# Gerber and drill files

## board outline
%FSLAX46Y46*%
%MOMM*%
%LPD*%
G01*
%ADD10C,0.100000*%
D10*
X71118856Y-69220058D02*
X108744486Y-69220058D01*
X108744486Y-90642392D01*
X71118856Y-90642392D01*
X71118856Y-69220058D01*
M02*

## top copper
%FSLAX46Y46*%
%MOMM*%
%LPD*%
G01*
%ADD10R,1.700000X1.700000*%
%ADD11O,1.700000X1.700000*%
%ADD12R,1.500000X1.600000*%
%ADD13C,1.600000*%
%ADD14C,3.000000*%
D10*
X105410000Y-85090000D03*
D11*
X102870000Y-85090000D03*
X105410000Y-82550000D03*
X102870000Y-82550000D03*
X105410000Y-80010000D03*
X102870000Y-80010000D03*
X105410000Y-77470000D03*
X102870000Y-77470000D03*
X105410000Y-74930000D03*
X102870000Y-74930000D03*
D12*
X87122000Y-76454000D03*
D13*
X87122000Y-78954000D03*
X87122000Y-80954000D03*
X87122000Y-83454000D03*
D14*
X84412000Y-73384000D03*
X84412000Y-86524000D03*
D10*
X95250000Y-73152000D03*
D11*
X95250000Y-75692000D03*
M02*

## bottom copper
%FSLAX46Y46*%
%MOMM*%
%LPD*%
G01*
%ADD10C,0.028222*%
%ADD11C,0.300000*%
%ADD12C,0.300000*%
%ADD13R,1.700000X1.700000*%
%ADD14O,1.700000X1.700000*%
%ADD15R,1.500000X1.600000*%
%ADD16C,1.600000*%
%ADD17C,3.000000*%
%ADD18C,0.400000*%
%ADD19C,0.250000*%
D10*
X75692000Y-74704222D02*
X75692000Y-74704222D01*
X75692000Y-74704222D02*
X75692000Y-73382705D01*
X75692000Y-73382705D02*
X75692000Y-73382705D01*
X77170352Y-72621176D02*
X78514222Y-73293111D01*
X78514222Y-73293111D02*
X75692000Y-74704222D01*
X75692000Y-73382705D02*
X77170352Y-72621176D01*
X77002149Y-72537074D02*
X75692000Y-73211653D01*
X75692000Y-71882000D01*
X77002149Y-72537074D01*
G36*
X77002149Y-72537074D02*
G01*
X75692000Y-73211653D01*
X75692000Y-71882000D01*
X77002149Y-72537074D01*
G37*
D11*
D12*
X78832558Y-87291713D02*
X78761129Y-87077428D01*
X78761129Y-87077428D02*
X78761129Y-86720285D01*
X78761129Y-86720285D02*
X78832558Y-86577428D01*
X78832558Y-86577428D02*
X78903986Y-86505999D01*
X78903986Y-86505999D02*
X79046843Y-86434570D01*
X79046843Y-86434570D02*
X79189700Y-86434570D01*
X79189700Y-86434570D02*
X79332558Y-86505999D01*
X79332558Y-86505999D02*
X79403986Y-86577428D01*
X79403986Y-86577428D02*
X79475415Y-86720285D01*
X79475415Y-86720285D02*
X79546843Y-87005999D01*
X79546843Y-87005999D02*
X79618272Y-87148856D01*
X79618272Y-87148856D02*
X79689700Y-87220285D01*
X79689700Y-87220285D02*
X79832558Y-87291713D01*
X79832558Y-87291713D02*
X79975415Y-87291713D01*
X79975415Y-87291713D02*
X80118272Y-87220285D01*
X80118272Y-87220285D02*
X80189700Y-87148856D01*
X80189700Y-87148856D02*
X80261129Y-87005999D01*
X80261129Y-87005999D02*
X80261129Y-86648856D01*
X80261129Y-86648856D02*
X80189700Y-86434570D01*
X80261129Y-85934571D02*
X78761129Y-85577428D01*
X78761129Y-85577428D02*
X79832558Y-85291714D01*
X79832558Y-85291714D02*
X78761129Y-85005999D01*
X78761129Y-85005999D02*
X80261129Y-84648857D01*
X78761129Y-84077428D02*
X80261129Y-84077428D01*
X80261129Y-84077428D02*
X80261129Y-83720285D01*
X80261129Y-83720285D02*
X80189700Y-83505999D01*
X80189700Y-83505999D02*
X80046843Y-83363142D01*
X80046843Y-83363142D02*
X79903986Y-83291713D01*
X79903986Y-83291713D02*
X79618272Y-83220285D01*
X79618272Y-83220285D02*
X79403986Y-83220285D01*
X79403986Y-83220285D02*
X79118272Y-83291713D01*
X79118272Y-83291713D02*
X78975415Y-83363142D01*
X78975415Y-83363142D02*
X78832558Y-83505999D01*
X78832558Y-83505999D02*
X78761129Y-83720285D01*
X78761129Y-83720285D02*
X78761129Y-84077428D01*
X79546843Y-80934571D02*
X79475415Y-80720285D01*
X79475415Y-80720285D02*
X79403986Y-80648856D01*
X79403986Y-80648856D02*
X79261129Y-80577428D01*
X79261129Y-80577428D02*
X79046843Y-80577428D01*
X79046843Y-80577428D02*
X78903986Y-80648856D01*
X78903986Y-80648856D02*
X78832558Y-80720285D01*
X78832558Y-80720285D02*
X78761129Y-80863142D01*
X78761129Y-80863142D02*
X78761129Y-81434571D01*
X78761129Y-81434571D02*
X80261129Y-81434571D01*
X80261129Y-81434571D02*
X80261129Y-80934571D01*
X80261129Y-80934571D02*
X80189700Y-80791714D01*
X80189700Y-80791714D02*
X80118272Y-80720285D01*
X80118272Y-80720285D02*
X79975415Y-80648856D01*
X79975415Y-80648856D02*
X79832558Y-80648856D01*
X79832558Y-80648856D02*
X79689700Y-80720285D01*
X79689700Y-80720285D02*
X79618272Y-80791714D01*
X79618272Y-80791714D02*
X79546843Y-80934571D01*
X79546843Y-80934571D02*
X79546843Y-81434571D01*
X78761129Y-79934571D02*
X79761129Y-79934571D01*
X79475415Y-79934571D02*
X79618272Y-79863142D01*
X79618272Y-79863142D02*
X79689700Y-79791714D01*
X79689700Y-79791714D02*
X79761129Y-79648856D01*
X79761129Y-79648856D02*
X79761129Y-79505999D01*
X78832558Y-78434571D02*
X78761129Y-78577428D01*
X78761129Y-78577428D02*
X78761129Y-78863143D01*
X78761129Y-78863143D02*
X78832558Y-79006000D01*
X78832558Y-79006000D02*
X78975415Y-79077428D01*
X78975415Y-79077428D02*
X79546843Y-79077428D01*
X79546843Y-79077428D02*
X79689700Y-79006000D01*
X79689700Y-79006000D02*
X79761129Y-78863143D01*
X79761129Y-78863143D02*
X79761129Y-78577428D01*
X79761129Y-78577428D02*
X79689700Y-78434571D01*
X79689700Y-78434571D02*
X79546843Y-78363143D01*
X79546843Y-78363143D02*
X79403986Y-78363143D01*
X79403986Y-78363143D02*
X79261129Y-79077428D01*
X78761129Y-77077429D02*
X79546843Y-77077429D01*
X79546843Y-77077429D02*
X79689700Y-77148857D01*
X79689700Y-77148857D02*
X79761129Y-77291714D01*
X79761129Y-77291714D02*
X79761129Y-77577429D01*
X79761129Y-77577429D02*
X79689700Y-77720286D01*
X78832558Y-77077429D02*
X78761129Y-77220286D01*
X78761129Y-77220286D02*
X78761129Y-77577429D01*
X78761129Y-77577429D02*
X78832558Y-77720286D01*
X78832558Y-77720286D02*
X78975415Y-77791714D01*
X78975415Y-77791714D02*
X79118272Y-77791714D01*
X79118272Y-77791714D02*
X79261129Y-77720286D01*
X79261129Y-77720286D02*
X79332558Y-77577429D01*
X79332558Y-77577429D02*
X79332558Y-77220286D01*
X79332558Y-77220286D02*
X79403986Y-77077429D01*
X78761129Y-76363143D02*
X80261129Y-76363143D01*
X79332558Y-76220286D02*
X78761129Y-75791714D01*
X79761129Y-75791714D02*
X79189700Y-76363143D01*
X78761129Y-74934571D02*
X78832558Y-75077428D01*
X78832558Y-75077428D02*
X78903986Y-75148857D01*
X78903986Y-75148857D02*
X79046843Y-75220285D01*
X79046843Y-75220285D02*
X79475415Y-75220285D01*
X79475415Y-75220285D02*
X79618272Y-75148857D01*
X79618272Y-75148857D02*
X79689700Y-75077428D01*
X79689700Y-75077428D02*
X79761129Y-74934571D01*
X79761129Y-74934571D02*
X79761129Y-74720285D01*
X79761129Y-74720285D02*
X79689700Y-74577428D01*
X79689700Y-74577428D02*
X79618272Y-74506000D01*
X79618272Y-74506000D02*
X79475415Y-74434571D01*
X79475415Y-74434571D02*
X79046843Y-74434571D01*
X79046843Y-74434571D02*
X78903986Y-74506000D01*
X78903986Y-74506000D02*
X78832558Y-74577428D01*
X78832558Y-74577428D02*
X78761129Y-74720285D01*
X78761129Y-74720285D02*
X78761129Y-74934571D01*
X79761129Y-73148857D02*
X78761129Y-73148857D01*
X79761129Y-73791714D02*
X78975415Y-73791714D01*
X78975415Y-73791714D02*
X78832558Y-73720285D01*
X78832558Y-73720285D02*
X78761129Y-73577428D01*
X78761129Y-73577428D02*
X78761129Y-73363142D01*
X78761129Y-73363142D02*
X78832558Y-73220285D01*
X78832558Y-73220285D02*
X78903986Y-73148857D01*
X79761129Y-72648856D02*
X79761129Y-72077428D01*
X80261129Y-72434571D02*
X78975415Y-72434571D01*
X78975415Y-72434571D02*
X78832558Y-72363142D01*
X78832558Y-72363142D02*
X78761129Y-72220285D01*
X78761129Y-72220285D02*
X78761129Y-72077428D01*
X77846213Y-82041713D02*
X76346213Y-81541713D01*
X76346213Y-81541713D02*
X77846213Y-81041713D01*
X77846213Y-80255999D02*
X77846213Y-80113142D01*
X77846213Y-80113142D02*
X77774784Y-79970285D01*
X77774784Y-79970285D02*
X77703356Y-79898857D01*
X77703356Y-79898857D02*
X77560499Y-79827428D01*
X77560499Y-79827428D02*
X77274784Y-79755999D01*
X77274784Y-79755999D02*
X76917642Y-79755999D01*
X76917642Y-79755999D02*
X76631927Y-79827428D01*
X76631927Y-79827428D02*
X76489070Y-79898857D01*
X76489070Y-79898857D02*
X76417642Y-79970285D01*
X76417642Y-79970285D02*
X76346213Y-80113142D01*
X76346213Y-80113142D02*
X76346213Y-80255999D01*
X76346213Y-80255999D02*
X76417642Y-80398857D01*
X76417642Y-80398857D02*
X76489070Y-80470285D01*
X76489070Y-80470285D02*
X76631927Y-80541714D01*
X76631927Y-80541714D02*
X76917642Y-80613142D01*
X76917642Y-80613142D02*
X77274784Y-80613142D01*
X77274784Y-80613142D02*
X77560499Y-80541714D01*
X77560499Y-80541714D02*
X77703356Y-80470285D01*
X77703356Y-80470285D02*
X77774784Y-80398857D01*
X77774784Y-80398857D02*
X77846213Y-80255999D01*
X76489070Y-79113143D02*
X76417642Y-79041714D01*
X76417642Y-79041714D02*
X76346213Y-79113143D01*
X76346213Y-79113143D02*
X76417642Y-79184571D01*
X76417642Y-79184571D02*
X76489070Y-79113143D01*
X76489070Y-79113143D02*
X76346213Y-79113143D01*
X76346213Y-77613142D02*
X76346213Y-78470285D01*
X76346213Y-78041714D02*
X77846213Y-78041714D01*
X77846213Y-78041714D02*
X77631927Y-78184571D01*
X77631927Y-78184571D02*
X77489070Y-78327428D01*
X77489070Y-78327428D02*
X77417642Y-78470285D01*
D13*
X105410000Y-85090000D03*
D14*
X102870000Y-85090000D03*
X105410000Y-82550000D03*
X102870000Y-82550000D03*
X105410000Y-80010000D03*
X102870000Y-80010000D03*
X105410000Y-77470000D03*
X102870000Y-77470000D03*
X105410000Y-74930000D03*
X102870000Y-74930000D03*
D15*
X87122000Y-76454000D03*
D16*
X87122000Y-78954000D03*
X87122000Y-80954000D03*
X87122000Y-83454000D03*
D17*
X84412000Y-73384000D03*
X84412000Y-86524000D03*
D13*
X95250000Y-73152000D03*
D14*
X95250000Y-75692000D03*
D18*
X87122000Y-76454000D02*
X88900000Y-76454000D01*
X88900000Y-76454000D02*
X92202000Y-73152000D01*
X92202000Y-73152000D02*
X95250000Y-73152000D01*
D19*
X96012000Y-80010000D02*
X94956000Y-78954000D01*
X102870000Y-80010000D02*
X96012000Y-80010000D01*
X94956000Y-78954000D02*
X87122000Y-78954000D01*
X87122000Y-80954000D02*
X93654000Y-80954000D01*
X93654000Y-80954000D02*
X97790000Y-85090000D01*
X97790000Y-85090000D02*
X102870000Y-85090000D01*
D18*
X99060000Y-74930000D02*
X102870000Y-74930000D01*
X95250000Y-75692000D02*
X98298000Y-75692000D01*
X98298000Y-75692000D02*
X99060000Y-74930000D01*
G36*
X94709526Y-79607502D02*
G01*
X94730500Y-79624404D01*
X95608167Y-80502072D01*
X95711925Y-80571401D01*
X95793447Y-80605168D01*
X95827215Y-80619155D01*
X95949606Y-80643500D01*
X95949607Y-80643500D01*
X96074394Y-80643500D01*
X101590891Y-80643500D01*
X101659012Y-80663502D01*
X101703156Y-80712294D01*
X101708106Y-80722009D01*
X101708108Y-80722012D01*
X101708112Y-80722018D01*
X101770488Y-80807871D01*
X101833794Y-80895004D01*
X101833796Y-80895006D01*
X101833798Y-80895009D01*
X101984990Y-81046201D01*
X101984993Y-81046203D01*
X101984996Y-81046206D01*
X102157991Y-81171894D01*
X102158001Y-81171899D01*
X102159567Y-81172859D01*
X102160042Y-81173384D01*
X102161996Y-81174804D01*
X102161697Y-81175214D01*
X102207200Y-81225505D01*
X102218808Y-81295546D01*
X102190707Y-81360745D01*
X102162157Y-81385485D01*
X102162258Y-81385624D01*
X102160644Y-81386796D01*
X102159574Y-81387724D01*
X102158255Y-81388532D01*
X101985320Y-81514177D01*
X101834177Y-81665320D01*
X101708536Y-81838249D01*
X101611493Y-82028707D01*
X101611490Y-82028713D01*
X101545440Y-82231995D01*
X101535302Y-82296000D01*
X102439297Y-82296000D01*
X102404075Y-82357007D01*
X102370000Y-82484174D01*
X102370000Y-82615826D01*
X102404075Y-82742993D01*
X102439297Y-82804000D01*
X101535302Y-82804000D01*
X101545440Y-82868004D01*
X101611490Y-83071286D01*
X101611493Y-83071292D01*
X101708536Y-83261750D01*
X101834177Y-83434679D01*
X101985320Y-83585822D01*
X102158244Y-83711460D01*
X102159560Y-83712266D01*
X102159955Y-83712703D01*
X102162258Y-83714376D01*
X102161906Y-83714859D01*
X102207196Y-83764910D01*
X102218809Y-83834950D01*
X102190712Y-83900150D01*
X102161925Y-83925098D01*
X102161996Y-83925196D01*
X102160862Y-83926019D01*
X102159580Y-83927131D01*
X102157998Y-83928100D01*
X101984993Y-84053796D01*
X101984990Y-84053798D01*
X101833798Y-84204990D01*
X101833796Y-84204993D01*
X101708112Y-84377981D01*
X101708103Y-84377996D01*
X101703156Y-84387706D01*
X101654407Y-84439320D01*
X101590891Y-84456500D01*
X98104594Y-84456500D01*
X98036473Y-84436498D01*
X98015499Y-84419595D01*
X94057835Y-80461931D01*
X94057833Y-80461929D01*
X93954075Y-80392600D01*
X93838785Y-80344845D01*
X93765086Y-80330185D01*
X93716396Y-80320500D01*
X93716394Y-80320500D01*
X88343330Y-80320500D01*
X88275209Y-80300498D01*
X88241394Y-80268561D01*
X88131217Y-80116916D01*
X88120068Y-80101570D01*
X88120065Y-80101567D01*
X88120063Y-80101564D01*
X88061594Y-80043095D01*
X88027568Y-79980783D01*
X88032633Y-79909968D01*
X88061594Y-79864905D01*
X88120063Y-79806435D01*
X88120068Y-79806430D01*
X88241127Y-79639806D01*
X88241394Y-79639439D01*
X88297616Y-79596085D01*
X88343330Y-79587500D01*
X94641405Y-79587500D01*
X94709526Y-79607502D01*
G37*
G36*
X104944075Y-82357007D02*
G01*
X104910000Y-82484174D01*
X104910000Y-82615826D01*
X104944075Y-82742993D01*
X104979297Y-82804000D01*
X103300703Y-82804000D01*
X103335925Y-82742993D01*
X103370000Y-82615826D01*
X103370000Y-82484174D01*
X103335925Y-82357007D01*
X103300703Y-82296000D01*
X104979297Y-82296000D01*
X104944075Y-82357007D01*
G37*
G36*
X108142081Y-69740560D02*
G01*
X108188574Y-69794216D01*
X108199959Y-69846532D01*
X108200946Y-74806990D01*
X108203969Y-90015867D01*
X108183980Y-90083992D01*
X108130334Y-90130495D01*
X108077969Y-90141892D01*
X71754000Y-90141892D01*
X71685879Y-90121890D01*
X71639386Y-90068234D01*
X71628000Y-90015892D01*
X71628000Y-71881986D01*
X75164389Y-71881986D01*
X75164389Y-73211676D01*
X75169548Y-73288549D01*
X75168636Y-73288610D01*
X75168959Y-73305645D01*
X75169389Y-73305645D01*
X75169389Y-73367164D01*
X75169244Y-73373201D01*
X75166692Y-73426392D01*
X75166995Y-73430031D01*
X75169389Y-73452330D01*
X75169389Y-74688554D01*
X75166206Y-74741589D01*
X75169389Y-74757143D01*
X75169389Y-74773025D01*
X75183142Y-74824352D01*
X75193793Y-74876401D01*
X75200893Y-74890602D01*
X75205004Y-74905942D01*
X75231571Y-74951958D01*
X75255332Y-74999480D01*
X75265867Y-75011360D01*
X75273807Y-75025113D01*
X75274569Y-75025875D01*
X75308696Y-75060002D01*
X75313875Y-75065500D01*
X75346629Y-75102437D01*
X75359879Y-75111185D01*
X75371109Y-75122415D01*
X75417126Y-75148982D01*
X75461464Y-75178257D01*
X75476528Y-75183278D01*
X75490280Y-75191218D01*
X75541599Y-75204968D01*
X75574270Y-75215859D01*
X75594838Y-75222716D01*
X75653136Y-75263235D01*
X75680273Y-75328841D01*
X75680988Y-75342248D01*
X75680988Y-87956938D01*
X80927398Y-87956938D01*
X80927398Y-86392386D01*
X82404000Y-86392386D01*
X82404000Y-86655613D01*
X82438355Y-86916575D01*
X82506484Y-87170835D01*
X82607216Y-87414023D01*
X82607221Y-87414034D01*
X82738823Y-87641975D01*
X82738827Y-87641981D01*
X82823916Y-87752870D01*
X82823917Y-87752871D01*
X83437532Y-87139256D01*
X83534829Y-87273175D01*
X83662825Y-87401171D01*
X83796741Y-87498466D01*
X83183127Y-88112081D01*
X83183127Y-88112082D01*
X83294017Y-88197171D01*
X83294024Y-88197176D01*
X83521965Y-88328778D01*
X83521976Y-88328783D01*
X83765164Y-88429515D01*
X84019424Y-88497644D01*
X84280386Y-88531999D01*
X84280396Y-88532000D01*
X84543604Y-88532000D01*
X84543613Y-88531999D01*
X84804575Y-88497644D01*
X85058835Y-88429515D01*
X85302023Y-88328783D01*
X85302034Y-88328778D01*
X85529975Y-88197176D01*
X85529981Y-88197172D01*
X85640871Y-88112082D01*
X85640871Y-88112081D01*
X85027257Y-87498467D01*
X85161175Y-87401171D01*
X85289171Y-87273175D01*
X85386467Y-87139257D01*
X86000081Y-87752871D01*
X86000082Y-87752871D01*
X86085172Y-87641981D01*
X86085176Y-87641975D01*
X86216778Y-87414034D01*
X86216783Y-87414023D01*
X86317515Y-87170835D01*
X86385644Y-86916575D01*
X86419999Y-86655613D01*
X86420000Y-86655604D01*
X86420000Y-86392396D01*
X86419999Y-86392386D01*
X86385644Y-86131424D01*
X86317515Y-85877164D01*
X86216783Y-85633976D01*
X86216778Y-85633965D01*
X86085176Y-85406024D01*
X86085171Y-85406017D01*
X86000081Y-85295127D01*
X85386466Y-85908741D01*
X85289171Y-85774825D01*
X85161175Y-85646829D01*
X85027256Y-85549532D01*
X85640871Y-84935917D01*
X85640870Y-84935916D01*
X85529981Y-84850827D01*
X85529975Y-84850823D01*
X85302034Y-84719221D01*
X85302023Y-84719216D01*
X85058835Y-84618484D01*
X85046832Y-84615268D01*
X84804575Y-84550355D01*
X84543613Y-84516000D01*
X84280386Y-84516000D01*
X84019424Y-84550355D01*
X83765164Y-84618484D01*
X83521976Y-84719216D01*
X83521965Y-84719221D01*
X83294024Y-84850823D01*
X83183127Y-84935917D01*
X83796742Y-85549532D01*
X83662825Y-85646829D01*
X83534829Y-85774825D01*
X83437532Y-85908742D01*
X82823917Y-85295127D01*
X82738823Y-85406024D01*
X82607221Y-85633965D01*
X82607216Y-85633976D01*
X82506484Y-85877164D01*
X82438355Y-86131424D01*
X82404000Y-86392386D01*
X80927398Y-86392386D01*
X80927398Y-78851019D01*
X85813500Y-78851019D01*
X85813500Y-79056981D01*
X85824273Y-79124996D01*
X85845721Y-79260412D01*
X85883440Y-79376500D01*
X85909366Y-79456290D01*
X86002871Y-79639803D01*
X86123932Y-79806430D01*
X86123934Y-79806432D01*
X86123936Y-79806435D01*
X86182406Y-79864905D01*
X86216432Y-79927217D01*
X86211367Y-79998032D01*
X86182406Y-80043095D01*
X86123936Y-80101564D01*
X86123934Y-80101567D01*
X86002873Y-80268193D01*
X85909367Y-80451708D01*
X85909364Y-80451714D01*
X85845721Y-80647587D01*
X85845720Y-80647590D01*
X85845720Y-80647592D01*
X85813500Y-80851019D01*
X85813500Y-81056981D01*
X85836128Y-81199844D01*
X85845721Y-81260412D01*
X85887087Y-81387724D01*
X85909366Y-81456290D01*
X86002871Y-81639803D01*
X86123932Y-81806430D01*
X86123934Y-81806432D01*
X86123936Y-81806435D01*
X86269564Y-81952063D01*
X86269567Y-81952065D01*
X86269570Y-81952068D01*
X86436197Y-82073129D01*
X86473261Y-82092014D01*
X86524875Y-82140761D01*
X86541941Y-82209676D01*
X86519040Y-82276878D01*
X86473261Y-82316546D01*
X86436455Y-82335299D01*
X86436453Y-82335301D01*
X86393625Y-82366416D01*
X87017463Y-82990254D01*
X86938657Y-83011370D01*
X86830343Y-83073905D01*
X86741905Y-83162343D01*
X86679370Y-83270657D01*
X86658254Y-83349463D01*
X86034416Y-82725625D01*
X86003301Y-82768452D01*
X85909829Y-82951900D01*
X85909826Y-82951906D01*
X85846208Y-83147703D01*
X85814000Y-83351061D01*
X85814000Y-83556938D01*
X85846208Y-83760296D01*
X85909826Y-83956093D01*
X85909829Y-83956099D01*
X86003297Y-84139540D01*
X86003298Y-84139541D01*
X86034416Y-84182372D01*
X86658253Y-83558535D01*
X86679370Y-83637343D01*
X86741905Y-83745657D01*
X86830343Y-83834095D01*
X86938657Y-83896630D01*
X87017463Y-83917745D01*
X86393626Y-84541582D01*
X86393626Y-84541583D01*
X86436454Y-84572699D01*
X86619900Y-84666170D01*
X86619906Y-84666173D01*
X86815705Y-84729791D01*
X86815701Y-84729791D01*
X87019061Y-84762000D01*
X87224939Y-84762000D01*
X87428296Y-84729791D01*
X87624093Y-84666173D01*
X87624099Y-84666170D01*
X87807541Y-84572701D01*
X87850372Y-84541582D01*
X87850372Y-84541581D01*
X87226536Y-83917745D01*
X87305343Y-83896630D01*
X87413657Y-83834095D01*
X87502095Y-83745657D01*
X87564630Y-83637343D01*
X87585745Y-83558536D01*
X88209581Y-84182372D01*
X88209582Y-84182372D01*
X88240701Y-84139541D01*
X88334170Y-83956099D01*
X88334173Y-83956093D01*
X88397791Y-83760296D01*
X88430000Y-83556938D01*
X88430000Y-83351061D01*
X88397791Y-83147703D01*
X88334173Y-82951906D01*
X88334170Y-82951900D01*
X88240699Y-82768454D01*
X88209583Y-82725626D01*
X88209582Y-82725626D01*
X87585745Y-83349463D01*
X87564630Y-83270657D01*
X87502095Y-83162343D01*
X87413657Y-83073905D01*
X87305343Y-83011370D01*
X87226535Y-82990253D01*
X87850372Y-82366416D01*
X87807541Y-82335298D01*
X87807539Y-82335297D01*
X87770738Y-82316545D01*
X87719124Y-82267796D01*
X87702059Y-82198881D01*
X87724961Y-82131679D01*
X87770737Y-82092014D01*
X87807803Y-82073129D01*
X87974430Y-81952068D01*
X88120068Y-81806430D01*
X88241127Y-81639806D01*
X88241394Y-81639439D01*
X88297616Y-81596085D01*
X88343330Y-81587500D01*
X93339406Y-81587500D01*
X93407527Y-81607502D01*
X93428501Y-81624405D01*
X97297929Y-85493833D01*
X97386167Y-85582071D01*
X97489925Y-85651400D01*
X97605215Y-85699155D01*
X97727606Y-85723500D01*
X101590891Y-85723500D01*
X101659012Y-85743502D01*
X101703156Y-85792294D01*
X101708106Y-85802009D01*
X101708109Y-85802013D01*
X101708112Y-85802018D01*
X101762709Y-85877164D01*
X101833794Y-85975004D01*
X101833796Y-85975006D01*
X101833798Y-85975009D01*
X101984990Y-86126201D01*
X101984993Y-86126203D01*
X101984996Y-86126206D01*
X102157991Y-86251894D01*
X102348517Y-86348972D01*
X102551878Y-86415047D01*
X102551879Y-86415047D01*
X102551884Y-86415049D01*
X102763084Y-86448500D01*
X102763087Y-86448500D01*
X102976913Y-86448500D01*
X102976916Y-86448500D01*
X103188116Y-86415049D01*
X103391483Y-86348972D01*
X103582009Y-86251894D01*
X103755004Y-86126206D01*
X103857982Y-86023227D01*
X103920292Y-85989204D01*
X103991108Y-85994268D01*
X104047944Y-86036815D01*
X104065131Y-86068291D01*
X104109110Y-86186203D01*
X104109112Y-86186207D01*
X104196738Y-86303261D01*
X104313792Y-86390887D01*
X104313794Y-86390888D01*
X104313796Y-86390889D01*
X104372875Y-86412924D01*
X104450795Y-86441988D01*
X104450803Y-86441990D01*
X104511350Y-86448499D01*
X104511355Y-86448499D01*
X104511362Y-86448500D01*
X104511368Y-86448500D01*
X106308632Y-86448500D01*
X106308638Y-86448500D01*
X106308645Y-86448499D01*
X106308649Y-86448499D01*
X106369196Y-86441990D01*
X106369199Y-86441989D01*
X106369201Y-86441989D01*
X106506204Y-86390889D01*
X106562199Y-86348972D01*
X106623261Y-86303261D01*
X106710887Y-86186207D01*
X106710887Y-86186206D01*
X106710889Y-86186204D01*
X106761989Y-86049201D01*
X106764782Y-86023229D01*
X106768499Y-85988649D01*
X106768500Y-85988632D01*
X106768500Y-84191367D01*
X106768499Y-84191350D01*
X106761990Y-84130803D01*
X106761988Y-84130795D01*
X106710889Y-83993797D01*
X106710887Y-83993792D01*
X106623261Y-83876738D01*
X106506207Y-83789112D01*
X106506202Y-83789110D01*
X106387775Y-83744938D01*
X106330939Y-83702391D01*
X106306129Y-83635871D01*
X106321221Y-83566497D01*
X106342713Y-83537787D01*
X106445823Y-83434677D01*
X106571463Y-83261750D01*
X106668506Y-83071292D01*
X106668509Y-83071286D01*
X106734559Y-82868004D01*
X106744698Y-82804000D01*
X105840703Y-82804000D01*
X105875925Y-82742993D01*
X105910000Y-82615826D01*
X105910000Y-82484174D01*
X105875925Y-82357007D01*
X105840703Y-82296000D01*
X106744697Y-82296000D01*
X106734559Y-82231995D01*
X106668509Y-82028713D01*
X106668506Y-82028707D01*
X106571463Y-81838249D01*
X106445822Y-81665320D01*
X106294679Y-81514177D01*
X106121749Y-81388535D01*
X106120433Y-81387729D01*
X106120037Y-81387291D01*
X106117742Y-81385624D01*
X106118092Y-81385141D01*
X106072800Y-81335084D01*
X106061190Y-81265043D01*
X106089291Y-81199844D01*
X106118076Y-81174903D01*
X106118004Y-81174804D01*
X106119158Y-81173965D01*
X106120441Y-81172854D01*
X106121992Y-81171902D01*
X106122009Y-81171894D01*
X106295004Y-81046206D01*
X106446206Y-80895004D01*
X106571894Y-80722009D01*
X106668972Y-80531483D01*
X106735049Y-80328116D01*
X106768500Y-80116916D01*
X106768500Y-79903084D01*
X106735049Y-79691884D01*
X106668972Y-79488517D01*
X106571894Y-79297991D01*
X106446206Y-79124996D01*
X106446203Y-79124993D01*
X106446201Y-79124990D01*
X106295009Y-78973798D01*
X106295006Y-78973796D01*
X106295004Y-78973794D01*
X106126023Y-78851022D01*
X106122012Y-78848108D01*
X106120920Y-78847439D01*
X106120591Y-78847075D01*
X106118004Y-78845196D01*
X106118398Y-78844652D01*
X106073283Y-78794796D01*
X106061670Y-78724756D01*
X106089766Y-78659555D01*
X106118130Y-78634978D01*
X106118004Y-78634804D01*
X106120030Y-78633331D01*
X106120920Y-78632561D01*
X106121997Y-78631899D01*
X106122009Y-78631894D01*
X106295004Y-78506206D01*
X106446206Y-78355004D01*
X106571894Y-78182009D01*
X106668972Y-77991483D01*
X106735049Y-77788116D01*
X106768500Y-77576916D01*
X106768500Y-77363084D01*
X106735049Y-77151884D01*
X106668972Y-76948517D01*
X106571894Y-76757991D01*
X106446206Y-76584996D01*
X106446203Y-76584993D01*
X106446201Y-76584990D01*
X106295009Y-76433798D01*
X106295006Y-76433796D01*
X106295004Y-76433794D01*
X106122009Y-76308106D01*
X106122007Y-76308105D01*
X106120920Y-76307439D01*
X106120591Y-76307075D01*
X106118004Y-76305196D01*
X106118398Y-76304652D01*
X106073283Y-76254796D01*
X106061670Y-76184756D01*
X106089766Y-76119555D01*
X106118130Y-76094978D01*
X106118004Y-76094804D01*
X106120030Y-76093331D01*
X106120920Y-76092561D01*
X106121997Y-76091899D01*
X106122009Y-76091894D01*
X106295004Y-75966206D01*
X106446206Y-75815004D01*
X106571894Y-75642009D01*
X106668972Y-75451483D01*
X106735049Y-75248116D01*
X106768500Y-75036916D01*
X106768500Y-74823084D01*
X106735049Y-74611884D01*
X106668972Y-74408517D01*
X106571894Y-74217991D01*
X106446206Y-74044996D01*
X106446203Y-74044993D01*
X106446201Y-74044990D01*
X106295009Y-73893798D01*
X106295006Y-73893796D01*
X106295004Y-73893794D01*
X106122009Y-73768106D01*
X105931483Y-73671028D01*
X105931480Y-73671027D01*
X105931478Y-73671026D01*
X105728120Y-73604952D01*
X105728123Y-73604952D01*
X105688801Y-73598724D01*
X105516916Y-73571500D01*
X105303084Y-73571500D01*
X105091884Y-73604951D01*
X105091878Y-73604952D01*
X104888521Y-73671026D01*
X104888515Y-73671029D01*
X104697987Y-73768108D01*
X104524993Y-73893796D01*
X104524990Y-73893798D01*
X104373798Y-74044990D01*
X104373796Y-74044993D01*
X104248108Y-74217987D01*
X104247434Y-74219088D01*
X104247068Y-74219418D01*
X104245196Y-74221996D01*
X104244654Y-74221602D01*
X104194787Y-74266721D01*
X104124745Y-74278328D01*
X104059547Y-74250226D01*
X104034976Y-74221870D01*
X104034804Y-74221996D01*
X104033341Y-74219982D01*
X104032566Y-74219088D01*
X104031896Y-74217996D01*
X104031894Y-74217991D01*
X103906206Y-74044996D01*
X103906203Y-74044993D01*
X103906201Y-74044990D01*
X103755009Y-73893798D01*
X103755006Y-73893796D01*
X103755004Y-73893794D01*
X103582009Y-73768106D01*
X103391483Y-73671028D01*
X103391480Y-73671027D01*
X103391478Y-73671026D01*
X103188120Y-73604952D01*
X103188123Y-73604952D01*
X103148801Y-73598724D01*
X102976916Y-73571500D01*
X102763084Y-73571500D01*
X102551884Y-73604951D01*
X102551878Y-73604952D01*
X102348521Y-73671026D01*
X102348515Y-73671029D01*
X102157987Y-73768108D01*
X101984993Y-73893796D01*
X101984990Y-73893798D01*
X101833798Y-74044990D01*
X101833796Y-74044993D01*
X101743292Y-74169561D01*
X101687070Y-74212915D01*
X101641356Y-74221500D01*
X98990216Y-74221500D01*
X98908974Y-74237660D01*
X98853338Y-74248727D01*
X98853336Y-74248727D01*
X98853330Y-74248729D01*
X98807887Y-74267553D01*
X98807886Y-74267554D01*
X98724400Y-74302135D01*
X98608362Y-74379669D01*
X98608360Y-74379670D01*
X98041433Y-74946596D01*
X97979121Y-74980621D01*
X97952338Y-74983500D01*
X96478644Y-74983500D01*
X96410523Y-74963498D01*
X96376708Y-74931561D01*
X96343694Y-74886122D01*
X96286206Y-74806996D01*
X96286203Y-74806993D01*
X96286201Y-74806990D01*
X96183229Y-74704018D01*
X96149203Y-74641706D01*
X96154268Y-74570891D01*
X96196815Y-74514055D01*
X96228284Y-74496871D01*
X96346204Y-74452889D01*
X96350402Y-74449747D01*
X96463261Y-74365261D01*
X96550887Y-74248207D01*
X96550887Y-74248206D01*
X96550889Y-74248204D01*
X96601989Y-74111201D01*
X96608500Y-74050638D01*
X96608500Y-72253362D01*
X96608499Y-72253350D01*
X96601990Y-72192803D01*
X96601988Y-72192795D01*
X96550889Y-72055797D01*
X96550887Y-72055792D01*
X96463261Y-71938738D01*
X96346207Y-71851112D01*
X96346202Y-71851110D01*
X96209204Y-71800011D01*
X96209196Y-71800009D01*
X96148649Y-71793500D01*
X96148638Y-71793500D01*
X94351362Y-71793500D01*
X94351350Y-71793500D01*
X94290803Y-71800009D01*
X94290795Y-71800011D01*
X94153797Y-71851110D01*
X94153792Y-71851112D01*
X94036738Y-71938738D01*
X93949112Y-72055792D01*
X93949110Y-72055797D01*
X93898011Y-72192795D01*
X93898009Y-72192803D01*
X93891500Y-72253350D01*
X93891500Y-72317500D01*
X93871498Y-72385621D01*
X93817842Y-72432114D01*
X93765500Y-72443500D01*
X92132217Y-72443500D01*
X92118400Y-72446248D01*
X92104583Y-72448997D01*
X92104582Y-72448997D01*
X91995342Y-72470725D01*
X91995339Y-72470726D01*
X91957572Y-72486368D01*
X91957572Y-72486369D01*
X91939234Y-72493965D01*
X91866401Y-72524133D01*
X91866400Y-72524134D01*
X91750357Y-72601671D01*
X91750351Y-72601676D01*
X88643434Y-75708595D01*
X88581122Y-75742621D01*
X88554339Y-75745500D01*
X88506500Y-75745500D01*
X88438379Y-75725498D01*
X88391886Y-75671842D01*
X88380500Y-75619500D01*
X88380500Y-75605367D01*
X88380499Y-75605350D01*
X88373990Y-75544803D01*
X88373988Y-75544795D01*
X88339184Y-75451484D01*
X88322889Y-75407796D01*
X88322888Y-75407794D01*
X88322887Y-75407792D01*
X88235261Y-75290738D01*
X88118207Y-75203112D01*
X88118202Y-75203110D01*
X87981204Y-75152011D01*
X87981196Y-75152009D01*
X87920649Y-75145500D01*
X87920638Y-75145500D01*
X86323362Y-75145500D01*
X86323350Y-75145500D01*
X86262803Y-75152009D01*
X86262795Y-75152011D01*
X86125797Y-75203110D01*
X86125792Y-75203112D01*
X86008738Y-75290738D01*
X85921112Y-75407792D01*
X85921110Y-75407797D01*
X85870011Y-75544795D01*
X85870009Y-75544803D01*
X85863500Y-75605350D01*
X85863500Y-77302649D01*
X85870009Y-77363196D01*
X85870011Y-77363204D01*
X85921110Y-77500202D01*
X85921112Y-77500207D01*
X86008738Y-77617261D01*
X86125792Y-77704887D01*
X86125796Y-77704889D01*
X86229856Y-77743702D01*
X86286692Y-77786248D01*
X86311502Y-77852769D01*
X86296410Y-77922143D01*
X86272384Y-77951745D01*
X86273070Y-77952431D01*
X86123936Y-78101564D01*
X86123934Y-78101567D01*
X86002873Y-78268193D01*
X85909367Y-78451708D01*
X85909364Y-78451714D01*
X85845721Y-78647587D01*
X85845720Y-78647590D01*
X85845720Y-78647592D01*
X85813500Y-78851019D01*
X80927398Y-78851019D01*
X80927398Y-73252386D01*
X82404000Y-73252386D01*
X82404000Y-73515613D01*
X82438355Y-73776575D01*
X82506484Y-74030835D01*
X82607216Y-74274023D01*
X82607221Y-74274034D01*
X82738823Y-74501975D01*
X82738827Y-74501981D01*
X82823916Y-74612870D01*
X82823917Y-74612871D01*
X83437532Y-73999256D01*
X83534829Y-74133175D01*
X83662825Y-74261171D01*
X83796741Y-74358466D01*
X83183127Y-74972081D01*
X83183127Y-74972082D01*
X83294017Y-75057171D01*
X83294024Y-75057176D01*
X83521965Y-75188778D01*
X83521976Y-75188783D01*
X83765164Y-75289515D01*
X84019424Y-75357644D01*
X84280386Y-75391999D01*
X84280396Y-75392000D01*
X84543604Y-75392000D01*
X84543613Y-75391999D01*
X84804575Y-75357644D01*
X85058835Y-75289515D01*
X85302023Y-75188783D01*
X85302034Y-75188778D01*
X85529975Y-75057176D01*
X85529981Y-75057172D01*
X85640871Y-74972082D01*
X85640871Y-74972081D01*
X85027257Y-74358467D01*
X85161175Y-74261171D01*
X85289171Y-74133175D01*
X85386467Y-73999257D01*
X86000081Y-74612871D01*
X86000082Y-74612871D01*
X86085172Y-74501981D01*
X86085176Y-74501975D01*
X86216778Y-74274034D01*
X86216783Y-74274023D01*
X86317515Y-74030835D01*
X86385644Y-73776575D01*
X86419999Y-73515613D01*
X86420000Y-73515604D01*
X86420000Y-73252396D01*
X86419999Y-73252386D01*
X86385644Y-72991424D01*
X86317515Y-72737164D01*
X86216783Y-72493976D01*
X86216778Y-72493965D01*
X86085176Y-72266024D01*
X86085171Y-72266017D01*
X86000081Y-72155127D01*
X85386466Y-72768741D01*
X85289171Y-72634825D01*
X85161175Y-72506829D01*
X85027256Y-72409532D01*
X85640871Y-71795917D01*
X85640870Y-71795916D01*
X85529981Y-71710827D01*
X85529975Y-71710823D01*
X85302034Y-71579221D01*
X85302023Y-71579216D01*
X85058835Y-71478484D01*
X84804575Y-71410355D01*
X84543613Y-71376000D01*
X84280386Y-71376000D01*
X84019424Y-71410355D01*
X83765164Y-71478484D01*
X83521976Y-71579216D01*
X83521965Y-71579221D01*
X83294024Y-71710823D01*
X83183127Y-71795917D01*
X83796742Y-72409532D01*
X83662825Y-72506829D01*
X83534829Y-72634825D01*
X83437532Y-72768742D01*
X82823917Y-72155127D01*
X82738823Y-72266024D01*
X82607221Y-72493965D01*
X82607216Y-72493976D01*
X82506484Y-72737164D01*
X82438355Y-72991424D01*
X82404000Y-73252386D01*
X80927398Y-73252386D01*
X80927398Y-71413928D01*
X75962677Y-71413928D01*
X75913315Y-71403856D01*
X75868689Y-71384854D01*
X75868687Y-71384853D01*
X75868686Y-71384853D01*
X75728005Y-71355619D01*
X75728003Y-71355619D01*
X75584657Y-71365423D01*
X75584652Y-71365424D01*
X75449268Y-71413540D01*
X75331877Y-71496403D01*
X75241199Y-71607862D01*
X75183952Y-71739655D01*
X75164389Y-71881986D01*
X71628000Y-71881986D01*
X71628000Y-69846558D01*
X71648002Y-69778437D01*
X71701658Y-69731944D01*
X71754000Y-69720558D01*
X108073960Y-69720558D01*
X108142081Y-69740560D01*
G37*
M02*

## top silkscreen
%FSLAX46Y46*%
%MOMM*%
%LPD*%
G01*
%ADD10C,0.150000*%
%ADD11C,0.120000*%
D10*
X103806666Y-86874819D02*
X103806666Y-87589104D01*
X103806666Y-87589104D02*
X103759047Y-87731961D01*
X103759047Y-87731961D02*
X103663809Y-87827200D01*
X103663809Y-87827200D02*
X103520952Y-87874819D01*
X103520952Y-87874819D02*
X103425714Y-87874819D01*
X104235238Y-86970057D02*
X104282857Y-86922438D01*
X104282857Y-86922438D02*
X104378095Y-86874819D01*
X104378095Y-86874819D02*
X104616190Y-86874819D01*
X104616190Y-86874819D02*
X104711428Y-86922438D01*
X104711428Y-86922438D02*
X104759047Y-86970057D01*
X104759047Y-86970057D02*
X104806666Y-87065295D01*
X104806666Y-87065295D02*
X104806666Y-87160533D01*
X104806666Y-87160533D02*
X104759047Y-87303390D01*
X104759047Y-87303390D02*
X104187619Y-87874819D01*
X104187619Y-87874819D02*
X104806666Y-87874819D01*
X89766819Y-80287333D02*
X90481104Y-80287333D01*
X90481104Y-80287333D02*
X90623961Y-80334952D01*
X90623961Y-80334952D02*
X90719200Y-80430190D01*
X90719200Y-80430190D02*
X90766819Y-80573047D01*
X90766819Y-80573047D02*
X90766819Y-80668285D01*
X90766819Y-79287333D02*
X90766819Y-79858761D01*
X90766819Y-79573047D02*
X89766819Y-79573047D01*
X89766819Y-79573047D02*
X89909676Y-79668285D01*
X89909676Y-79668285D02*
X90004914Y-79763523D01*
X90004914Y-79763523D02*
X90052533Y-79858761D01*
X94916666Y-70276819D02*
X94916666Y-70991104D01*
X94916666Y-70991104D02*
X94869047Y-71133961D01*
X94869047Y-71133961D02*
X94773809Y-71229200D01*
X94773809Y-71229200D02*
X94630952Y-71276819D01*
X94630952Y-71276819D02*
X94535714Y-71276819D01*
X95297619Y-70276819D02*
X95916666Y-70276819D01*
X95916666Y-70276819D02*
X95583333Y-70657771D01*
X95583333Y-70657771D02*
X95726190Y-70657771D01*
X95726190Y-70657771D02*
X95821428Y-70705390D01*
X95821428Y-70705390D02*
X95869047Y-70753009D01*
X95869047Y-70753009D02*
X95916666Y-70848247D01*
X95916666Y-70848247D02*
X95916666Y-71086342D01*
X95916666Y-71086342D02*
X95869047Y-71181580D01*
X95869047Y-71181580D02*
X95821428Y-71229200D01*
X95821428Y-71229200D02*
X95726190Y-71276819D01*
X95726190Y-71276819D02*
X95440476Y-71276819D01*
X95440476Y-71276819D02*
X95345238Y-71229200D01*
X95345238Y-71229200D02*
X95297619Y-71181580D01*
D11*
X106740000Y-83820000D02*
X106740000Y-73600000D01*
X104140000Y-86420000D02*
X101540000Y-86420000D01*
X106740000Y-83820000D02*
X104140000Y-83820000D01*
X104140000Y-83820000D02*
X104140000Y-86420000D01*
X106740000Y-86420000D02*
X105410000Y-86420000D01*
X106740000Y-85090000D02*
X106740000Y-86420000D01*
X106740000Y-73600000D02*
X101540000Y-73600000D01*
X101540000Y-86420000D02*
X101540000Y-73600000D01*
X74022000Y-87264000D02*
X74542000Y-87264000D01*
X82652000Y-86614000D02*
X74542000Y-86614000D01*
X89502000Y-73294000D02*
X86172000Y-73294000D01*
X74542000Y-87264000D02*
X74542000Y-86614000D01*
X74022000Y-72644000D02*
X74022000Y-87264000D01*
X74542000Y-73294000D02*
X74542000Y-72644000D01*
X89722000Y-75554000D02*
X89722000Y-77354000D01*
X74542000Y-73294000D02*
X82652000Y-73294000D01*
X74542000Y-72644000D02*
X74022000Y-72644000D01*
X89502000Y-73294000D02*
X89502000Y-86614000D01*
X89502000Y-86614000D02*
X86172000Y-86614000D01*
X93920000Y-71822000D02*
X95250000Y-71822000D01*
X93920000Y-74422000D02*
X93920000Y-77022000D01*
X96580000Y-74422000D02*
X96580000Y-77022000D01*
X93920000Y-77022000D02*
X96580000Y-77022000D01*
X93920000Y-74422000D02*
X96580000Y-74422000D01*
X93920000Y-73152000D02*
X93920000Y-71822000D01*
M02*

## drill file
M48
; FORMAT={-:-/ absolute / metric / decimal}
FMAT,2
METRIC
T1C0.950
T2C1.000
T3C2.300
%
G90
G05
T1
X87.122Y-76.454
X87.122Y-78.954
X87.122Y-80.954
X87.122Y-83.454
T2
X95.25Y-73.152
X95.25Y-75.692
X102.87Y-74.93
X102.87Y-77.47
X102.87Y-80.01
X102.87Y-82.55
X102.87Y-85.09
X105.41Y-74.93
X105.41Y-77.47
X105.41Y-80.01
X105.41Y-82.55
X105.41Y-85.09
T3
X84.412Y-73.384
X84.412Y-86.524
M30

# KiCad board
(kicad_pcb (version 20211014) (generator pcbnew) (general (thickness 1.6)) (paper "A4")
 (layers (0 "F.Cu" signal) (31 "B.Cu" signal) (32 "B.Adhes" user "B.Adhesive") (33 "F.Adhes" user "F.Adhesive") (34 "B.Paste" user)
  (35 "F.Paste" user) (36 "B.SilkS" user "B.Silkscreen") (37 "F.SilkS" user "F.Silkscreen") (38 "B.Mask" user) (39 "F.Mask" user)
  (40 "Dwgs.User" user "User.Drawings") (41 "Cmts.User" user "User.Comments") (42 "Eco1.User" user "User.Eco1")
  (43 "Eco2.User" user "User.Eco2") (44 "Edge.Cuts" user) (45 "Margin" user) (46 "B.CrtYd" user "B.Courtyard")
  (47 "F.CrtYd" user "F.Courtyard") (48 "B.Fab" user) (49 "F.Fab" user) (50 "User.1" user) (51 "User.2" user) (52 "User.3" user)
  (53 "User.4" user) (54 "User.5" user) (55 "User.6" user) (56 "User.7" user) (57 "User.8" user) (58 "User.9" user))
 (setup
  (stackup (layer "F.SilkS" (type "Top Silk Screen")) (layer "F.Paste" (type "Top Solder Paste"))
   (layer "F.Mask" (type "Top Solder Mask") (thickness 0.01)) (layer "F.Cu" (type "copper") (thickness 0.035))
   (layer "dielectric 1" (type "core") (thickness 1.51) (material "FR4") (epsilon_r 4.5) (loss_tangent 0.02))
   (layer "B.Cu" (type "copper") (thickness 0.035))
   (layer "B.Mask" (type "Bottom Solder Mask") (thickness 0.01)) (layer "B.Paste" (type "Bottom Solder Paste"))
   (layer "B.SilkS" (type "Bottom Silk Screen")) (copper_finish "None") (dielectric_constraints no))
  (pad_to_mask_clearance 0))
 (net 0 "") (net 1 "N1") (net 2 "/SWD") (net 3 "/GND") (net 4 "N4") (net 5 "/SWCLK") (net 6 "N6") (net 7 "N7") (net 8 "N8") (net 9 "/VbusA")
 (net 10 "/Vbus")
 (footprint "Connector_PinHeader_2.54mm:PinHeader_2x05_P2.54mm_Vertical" (layer "F.Cu") (at 105.41 85.09 180)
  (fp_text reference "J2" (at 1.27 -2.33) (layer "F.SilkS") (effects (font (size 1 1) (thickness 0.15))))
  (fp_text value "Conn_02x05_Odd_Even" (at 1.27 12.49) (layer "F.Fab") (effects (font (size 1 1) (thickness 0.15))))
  (fp_line (start -1.33 1.27) (end -1.33 11.49) (layer "F.SilkS") (width 0.12))
  (fp_line (start 1.27 -1.33) (end 3.87 -1.33) (layer "F.SilkS") (width 0.12))
  (fp_line (start -1.33 1.27) (end 1.27 1.27) (layer "F.SilkS") (width 0.12))
  (fp_line (start 1.27 1.27) (end 1.27 -1.33) (layer "F.SilkS") (width 0.12))
  (fp_line (start -1.33 -1.33) (end 0 -1.33) (layer "F.SilkS") (width 0.12))
  (fp_line (start -1.33 0) (end -1.33 -1.33) (layer "F.SilkS") (width 0.12))
  (fp_line (start -1.33 11.49) (end 3.87 11.49) (layer "F.SilkS") (width 0.12))
  (fp_line (start 3.87 -1.33) (end 3.87 11.49) (layer "F.SilkS") (width 0.12))
  (pad "1" thru_hole rect (at 0 0 180) (size 1.7 1.7) (drill 1) (layers *.Cu *.Mask) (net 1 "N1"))
  (pad "2" thru_hole oval (at 2.54 0 180) (size 1.7 1.7) (drill 1) (layers *.Cu *.Mask) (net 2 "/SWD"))
  (pad "3" thru_hole oval (at 0 2.54 180) (size 1.7 1.7) (drill 1) (layers *.Cu *.Mask) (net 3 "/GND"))
  (pad "4" thru_hole oval (at 2.54 2.54 180) (size 1.7 1.7) (drill 1) (layers *.Cu *.Mask) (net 3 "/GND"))
  (pad "5" thru_hole oval (at 0 5.08 180) (size 1.7 1.7) (drill 1) (layers *.Cu *.Mask) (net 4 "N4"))
  (pad "6" thru_hole oval (at 2.54 5.08 180) (size 1.7 1.7) (drill 1) (layers *.Cu *.Mask) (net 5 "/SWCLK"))
  (pad "7" thru_hole oval (at 0 7.62 180) (size 1.7 1.7) (drill 1) (layers *.Cu *.Mask) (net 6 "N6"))
  (pad "8" thru_hole oval (at 2.54 7.62 180) (size 1.7 1.7) (drill 1) (layers *.Cu *.Mask) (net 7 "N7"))
  (pad "9" thru_hole oval (at 0 10.16 180) (size 1.7 1.7) (drill 1) (layers *.Cu *.Mask) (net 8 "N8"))
  (pad "10" thru_hole oval (at 2.54 10.16 180) (size 1.7 1.7) (drill 1) (layers *.Cu *.Mask) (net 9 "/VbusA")))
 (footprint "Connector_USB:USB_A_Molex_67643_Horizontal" (layer "F.Cu") (at 87.122 76.454 -90)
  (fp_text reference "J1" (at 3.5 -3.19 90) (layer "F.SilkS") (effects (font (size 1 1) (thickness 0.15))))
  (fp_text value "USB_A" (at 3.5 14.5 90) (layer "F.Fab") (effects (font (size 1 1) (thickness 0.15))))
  (fp_line (start 10.81 13.1) (end 10.81 12.58) (layer "F.SilkS") (width 0.12))
  (fp_line (start 10.16 4.47) (end 10.16 12.58) (layer "F.SilkS") (width 0.12))
  (fp_line (start -3.16 -2.38) (end -3.16 0.95) (layer "F.SilkS") (width 0.12))
  (fp_line (start 10.81 12.58) (end 10.16 12.58) (layer "F.SilkS") (width 0.12))
  (fp_line (start -3.81 13.1) (end 10.81 13.1) (layer "F.SilkS") (width 0.12))
  (fp_line (start -3.16 12.58) (end -3.81 12.58) (layer "F.SilkS") (width 0.12))
  (fp_line (start -0.9 -2.6) (end 0.9 -2.6) (layer "F.SilkS") (width 0.12))
  (fp_line (start -3.16 12.58) (end -3.16 4.47) (layer "F.SilkS") (width 0.12))
  (fp_line (start -3.81 12.58) (end -3.81 13.1) (layer "F.SilkS") (width 0.12))
  (fp_line (start -3.16 -2.38) (end 10.16 -2.38) (layer "F.SilkS") (width 0.12))
  (fp_line (start 10.16 -2.38) (end 10.16 0.95) (layer "F.SilkS") (width 0.12))
  (pad "1" thru_hole rect (at 0 0 270) (size 1.6 1.5) (drill 0.95) (layers *.Cu *.Mask) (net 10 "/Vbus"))
  (pad "2" thru_hole circle (at 2.5 0 270) (size 1.6 1.6) (drill 0.95) (layers *.Cu *.Mask) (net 5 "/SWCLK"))
  (pad "3" thru_hole circle (at 4.5 0 270) (size 1.6 1.6) (drill 0.95) (layers *.Cu *.Mask) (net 2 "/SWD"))
  (pad "4" thru_hole circle (at 7 0 270) (size 1.6 1.6) (drill 0.95) (layers *.Cu *.Mask) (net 3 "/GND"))
  (pad "5" thru_hole circle (at -3.07 2.71 270) (size 3 3) (drill 2.3) (layers *.Cu *.Mask) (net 3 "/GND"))
  (pad "5" thru_hole circle (at 10.07 2.71 270) (size 3 3) (drill 2.3) (layers *.Cu *.Mask) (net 3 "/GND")))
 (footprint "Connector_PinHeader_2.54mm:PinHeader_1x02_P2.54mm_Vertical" (layer "F.Cu") (at 95.25 73.152)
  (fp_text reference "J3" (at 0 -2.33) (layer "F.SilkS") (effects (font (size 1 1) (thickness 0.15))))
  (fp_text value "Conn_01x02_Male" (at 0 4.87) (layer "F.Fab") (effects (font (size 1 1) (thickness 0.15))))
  (fp_line (start -1.33 -1.33) (end 0 -1.33) (layer "F.SilkS") (width 0.12))
  (fp_line (start -1.33 1.27) (end -1.33 3.87) (layer "F.SilkS") (width 0.12))
  (fp_line (start 1.33 1.27) (end 1.33 3.87) (layer "F.SilkS") (width 0.12))
  (fp_line (start -1.33 3.87) (end 1.33 3.87) (layer "F.SilkS") (width 0.12))
  (fp_line (start -1.33 1.27) (end 1.33 1.27) (layer "F.SilkS") (width 0.12))
  (fp_line (start -1.33 0) (end -1.33 -1.33) (layer "F.SilkS") (width 0.12))
  (pad "1" thru_hole rect (at 0 0) (size 1.7 1.7) (drill 1) (layers *.Cu *.Mask) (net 10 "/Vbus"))
  (pad "2" thru_hole oval (at 0 2.54) (size 1.7 1.7) (drill 1) (layers *.Cu *.Mask) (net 9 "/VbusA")))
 (gr_line (start 75.692 74.704222) (end 75.692 74.704222) (layer "B.Cu") (width 0.028222))
 (gr_line (start 75.692 74.704222) (end 75.692 73.382705) (layer "B.Cu") (width 0.028222))
 (gr_line (start 75.692 73.382705) (end 75.692 73.382705) (layer "B.Cu") (width 0.028222))
 (gr_line (start 77.170352 72.621176) (end 78.514222 73.293111) (layer "B.Cu") (width 0.028222))
 (gr_line (start 78.514222 73.293111) (end 75.692 74.704222) (layer "B.Cu") (width 0.028222))
 (gr_line (start 75.692 73.382705) (end 77.170352 72.621176) (layer "B.Cu") (width 0.028222))
 (gr_poly
  (pts (xy 77.002149 72.537074) (xy 75.692 73.211653) (xy 75.692 71.882) (xy 77.002149 72.537074)) (layer "B.Cu") (width 0.028222)
  (fill solid))
 (gr_rect (start 71.118856 69.220058) (end 108.744486 90.642392) (layer "Edge.Cuts") (width 0.1) (fill none))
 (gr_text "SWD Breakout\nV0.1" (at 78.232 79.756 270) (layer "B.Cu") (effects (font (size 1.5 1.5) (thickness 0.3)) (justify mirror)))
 (segment (start 87.122 76.454) (end 88.9 76.454) (width 0.4) (layer "B.Cu") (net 10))
 (segment (start 88.9 76.454) (end 92.202 73.152) (width 0.4) (layer "B.Cu") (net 10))
 (segment (start 92.202 73.152) (end 95.25 73.152) (width 0.4) (layer "B.Cu") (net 10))
 (segment (start 96.012 80.01) (end 94.956 78.954) (width 0.25) (layer "B.Cu") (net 5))
 (segment (start 102.87 80.01) (end 96.012 80.01) (width 0.25) (layer "B.Cu") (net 5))
 (segment (start 94.956 78.954) (end 87.122 78.954) (width 0.25) (layer "B.Cu") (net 5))
 (segment (start 87.122 80.954) (end 93.654 80.954) (width 0.25) (layer "B.Cu") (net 2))
 (segment (start 93.654 80.954) (end 97.79 85.09) (width 0.25) (layer "B.Cu") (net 2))
 (segment (start 97.79 85.09) (end 102.87 85.09) (width 0.25) (layer "B.Cu") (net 2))
 (segment (start 99.06 74.93) (end 102.87 74.93) (width 0.4) (layer "B.Cu") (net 9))
 (segment (start 95.25 75.692) (end 98.298 75.692) (width 0.4) (layer "B.Cu") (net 9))
 (segment (start 98.298 75.692) (end 99.06 74.93) (width 0.4) (layer "B.Cu") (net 9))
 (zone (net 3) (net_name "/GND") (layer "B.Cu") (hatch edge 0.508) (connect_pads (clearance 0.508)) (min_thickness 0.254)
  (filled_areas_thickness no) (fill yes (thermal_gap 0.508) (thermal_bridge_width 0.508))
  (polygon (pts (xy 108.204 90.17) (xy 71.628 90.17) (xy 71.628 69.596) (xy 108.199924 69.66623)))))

